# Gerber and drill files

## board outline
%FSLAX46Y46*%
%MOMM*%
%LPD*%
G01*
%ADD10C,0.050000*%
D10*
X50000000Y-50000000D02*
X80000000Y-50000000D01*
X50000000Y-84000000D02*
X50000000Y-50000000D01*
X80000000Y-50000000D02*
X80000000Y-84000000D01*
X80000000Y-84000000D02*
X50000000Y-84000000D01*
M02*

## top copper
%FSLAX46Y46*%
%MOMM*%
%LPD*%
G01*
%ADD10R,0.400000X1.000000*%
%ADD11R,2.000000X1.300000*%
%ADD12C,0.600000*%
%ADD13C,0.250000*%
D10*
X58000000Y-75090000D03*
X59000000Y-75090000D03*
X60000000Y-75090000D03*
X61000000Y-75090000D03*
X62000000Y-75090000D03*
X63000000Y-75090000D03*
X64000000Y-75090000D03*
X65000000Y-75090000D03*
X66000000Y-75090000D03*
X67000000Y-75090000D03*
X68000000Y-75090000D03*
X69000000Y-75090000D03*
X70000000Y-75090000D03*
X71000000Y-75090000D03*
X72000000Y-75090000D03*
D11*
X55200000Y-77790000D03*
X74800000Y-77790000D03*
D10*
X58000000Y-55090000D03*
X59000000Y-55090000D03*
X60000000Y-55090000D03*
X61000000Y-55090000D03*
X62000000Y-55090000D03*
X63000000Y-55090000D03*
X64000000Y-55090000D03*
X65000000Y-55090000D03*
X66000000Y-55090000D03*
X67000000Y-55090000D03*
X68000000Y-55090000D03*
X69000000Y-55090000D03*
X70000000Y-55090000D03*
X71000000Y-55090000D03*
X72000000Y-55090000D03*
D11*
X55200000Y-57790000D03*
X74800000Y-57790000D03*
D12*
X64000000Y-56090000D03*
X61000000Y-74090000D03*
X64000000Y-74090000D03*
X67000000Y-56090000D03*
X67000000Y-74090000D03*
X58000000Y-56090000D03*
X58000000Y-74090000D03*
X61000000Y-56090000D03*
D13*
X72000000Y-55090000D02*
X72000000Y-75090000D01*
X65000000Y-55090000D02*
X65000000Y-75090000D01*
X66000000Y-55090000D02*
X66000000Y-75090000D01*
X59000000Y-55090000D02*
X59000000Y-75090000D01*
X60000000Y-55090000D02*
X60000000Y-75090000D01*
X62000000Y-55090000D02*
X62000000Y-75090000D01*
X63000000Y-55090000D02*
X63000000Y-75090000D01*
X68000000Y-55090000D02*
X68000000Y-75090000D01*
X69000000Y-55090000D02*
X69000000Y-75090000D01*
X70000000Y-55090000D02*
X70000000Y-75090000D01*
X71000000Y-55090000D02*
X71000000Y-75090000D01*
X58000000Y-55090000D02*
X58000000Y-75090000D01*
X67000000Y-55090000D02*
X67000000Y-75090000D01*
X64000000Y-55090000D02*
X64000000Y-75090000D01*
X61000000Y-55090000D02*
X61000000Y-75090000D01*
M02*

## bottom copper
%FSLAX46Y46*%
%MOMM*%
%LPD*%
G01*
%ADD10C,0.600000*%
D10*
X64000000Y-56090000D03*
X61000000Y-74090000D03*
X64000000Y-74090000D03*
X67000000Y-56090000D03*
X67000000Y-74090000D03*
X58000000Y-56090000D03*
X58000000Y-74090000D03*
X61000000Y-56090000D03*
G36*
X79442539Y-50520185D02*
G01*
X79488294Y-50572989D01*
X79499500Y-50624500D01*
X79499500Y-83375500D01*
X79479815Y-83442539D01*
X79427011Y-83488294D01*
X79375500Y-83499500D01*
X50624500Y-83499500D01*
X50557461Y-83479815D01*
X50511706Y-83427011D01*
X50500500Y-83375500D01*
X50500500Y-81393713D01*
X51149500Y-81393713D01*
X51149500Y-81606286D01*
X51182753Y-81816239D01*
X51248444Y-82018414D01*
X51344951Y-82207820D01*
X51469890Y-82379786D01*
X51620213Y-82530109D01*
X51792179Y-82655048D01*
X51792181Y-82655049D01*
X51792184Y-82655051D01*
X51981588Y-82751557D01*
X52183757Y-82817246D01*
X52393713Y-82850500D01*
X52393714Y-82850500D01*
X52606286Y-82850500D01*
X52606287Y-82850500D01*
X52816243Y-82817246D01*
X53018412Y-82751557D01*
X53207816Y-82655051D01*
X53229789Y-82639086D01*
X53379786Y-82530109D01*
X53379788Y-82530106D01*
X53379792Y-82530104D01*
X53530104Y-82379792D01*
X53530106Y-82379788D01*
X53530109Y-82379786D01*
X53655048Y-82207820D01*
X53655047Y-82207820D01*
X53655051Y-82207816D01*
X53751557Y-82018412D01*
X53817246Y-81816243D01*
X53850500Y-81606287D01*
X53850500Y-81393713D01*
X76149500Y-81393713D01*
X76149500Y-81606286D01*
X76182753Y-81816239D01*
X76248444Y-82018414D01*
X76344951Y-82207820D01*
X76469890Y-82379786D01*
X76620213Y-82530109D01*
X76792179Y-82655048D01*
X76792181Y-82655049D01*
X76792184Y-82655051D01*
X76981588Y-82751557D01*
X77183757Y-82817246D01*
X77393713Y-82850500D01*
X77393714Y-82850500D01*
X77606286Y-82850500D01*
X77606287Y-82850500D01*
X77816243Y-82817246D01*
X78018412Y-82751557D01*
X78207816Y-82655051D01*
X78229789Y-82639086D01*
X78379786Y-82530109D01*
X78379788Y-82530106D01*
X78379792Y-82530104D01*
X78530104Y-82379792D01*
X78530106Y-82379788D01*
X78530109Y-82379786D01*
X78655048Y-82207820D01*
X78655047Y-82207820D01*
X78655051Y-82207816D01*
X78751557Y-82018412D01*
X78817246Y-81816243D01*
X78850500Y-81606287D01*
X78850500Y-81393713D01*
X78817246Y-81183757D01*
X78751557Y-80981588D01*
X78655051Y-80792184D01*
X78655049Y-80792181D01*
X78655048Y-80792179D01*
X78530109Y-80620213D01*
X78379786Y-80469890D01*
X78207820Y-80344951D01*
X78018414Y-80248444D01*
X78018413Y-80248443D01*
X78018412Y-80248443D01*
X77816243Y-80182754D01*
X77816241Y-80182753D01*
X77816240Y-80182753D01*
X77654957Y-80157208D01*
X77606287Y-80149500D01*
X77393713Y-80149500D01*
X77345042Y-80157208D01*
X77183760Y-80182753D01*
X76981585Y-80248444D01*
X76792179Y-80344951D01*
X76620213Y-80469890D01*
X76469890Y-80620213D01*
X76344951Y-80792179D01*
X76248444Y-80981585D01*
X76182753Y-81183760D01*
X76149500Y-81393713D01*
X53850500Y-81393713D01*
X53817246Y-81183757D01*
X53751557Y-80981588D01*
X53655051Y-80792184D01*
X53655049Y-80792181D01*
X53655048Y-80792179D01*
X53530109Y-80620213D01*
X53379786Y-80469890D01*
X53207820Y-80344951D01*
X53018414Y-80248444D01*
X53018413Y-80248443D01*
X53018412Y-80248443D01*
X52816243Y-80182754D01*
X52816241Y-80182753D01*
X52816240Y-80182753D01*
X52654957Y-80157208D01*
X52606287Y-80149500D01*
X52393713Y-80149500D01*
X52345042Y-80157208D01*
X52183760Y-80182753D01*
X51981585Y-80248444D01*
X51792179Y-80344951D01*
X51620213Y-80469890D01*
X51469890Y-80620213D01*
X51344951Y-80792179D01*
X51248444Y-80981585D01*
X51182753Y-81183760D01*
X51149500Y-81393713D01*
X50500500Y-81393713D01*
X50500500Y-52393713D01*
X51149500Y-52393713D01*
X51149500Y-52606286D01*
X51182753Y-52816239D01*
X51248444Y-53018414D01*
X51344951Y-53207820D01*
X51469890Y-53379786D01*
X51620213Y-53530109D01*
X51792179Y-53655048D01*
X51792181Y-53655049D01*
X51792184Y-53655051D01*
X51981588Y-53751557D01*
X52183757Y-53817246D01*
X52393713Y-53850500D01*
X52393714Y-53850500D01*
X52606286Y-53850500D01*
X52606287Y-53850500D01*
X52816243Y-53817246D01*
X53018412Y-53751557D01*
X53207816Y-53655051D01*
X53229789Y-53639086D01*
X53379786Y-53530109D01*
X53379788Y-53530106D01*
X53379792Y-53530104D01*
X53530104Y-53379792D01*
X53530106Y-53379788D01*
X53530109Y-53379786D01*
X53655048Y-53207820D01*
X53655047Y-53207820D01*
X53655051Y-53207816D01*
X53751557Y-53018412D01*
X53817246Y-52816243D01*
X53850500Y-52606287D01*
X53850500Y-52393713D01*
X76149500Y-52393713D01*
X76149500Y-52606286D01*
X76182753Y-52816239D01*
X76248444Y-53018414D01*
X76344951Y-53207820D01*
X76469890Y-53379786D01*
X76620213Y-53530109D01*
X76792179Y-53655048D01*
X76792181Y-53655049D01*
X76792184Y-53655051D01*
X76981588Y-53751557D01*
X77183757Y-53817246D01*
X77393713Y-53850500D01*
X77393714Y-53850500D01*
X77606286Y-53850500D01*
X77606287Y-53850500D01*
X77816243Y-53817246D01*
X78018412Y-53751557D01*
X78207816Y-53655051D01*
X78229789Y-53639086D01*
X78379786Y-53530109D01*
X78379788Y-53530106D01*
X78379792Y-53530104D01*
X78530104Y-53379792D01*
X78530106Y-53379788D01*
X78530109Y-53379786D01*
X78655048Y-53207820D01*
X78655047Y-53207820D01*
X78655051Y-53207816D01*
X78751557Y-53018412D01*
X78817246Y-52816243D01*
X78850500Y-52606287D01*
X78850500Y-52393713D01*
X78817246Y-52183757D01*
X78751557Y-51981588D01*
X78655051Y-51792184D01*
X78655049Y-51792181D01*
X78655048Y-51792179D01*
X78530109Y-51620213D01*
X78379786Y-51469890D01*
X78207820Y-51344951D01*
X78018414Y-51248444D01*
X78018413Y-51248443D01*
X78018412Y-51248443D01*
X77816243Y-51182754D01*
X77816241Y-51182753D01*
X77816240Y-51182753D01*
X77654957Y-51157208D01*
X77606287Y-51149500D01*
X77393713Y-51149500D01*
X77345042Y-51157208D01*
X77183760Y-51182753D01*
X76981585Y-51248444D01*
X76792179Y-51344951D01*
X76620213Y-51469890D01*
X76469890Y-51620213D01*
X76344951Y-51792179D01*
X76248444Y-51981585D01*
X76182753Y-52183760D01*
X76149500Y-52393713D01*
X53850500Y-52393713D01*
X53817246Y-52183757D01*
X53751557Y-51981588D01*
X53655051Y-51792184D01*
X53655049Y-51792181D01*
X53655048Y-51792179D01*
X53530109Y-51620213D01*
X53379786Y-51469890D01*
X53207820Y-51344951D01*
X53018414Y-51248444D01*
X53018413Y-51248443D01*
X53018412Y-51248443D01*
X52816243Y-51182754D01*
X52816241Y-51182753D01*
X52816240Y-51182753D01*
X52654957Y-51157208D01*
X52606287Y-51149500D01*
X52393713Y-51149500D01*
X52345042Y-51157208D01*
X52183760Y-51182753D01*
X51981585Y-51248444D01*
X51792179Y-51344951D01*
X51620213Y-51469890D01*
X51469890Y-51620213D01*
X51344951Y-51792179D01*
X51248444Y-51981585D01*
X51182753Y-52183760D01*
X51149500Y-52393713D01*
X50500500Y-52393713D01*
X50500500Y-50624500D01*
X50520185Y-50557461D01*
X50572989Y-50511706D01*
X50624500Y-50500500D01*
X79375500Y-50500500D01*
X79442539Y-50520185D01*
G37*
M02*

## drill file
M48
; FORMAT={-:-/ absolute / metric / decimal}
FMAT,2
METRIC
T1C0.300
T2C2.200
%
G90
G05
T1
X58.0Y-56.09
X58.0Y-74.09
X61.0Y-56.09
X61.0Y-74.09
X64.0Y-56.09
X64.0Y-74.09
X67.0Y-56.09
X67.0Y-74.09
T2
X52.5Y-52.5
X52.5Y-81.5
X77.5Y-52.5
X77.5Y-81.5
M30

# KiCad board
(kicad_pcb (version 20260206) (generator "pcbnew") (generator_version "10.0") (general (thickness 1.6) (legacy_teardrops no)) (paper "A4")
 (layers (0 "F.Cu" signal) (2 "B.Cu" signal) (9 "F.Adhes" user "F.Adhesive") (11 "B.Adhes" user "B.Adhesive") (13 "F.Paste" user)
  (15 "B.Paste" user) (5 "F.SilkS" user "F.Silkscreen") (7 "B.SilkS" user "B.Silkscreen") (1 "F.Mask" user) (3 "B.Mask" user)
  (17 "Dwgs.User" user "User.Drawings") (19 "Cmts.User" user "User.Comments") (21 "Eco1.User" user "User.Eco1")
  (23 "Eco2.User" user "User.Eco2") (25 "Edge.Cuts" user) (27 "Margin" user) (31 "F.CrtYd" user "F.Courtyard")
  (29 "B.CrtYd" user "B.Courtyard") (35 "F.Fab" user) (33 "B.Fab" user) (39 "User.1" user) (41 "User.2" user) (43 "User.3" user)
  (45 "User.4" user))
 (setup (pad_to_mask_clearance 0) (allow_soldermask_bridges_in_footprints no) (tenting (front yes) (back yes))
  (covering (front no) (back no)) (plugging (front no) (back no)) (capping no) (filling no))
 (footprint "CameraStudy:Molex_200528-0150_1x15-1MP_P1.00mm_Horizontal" (layer "F.Cu") (at 65 76)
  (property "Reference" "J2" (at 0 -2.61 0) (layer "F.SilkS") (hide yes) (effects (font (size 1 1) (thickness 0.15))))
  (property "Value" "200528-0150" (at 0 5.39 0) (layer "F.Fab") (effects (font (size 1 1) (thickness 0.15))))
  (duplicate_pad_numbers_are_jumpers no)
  (pad "1" smd rect (at -7 -0.91) (size 0.4 1) (layers "F.Cu" "F.Mask" "F.Paste") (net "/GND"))
  (pad "2" smd rect (at -6 -0.91) (size 0.4 1) (layers "F.Cu" "F.Mask" "F.Paste") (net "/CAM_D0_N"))
  (pad "3" smd rect (at -5 -0.91) (size 0.4 1) (layers "F.Cu" "F.Mask" "F.Paste") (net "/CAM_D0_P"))
  (pad "4" smd rect (at -4 -0.91) (size 0.4 1) (layers "F.Cu" "F.Mask" "F.Paste") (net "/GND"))
  (pad "5" smd rect (at -3 -0.91) (size 0.4 1) (layers "F.Cu" "F.Mask" "F.Paste") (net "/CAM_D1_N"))
  (pad "6" smd rect (at -2 -0.91) (size 0.4 1) (layers "F.Cu" "F.Mask" "F.Paste") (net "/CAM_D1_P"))
  (pad "7" smd rect (at -1 -0.91) (size 0.4 1) (layers "F.Cu" "F.Mask" "F.Paste") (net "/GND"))
  (pad "8" smd rect (at 0 -0.91) (size 0.4 1) (layers "F.Cu" "F.Mask" "F.Paste") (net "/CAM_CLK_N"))
  (pad "9" smd rect (at 1 -0.91) (size 0.4 1) (layers "F.Cu" "F.Mask" "F.Paste") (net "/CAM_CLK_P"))
  (pad "10" smd rect (at 2 -0.91) (size 0.4 1) (layers "F.Cu" "F.Mask" "F.Paste") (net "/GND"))
  (pad "11" smd rect (at 3 -0.91) (size 0.4 1) (layers "F.Cu" "F.Mask" "F.Paste") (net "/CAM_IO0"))
  (pad "12" smd rect (at 4 -0.91) (size 0.4 1) (layers "F.Cu" "F.Mask" "F.Paste") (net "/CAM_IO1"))
  (pad "13" smd rect (at 5 -0.91) (size 0.4 1) (layers "F.Cu" "F.Mask" "F.Paste") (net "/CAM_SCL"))
  (pad "14" smd rect (at 6 -0.91) (size 0.4 1) (layers "F.Cu" "F.Mask" "F.Paste") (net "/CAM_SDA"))
  (pad "15" smd rect (at 7 -0.91) (size 0.4 1) (layers "F.Cu" "F.Mask" "F.Paste") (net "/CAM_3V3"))
  (pad "MP" smd rect (at -9.8 1.79) (size 2 1.3) (layers "F.Cu" "F.Mask" "F.Paste"))
  (pad "MP" smd rect (at 9.8 1.79) (size 2 1.3) (layers "F.Cu" "F.Mask" "F.Paste")))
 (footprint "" (layer "F.Cu") (at 77.5 52.5)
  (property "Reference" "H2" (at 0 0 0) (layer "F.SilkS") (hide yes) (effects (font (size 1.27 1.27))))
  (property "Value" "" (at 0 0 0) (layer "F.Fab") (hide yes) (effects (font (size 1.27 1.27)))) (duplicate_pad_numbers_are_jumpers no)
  (pad "" np_thru_hole circle (at 0 0) (size 2.2 2.2) (drill 2.2) (layers "*.Cu")))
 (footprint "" (layer "F.Cu") (at 77.5 81.5)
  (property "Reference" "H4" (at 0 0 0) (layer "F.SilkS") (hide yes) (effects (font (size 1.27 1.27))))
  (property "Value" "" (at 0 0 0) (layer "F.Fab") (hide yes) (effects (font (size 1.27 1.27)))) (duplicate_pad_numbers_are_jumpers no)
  (pad "" np_thru_hole circle (at 0 0) (size 2.2 2.2) (drill 2.2) (layers "*.Cu")))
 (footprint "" (layer "F.Cu") (at 52.5 52.5)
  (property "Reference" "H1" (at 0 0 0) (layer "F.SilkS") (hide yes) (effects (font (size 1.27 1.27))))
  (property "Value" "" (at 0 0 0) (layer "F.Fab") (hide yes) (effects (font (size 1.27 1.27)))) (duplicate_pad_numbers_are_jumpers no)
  (pad "" np_thru_hole circle (at 0 0) (size 2.2 2.2) (drill 2.2) (layers "*.Cu")))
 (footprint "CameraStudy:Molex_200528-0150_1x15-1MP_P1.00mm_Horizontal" (layer "F.Cu") (at 65 56)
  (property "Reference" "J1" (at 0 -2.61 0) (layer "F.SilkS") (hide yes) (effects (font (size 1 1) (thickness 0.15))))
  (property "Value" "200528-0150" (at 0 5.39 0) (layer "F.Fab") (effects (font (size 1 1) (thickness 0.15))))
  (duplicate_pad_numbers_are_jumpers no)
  (pad "1" smd rect (at -7 -0.91) (size 0.4 1) (layers "F.Cu" "F.Mask" "F.Paste") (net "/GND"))
  (pad "2" smd rect (at -6 -0.91) (size 0.4 1) (layers "F.Cu" "F.Mask" "F.Paste") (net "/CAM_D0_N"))
  (pad "3" smd rect (at -5 -0.91) (size 0.4 1) (layers "F.Cu" "F.Mask" "F.Paste") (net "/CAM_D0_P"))
  (pad "4" smd rect (at -4 -0.91) (size 0.4 1) (layers "F.Cu" "F.Mask" "F.Paste") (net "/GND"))
  (pad "5" smd rect (at -3 -0.91) (size 0.4 1) (layers "F.Cu" "F.Mask" "F.Paste") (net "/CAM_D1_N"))
  (pad "6" smd rect (at -2 -0.91) (size 0.4 1) (layers "F.Cu" "F.Mask" "F.Paste") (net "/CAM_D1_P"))
  (pad "7" smd rect (at -1 -0.91) (size 0.4 1) (layers "F.Cu" "F.Mask" "F.Paste") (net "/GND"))
  (pad "8" smd rect (at 0 -0.91) (size 0.4 1) (layers "F.Cu" "F.Mask" "F.Paste") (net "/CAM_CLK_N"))
  (pad "9" smd rect (at 1 -0.91) (size 0.4 1) (layers "F.Cu" "F.Mask" "F.Paste") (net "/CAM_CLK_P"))
  (pad "10" smd rect (at 2 -0.91) (size 0.4 1) (layers "F.Cu" "F.Mask" "F.Paste") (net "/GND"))
  (pad "11" smd rect (at 3 -0.91) (size 0.4 1) (layers "F.Cu" "F.Mask" "F.Paste") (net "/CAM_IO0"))
  (pad "12" smd rect (at 4 -0.91) (size 0.4 1) (layers "F.Cu" "F.Mask" "F.Paste") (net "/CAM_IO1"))
  (pad "13" smd rect (at 5 -0.91) (size 0.4 1) (layers "F.Cu" "F.Mask" "F.Paste") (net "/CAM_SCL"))
  (pad "14" smd rect (at 6 -0.91) (size 0.4 1) (layers "F.Cu" "F.Mask" "F.Paste") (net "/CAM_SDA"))
  (pad "15" smd rect (at 7 -0.91) (size 0.4 1) (layers "F.Cu" "F.Mask" "F.Paste") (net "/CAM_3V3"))
  (pad "MP" smd rect (at -9.8 1.79) (size 2 1.3) (layers "F.Cu" "F.Mask" "F.Paste"))
  (pad "MP" smd rect (at 9.8 1.79) (size 2 1.3) (layers "F.Cu" "F.Mask" "F.Paste")))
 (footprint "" (layer "F.Cu") (at 52.5 81.5)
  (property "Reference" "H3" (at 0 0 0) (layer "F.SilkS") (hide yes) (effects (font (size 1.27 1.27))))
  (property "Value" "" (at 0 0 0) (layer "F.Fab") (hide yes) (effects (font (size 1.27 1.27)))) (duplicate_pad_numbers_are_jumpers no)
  (pad "" np_thru_hole circle (at 0 0) (size 2.2 2.2) (drill 2.2) (layers "*.Cu")))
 (gr_line (start 50 50) (end 80 50) (stroke (width 0.05) (type default)) (layer "Edge.Cuts"))
 (gr_line (start 50 84) (end 50 50) (stroke (width 0.05) (type default)) (layer "Edge.Cuts"))
 (gr_line (start 80 50) (end 80 84) (stroke (width 0.05) (type default)) (layer "Edge.Cuts"))
 (gr_line (start 80 84) (end 50 84) (stroke (width 0.05) (type default)) (layer "Edge.Cuts"))
 (segment (start 72 55.09) (end 72 75.09) (width 0.25) (layer "F.Cu") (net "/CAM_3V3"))
 (segment (start 65 55.09) (end 65 75.09) (width 0.25) (layer "F.Cu") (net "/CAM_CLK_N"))
 (segment (start 66 55.09) (end 66 75.09) (width 0.25) (layer "F.Cu") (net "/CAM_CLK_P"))
 (segment (start 59 55.09) (end 59 75.09) (width 0.25) (layer "F.Cu") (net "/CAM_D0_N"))
 (segment (start 60 55.09) (end 60 75.09) (width 0.25) (layer "F.Cu") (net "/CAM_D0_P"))
 (segment (start 62 55.09) (end 62 75.09) (width 0.25) (layer "F.Cu") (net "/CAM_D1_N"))
 (segment (start 63 55.09) (end 63 75.09) (width 0.25) (layer "F.Cu") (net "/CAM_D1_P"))
 (segment (start 68 55.09) (end 68 75.09) (width 0.25) (layer "F.Cu") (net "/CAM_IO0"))
 (segment (start 69 55.09) (end 69 75.09) (width 0.25) (layer "F.Cu") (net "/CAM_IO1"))
 (segment (start 70 55.09) (end 70 75.09) (width 0.25) (layer "F.Cu") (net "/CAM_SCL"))
 (segment (start 71 55.09) (end 71 75.09) (width 0.25) (layer "F.Cu") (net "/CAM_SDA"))
 (segment (start 58 55.09) (end 58 75.09) (width 0.25) (layer "F.Cu") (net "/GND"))
 (segment (start 67 55.09) (end 67 75.09) (width 0.25) (layer "F.Cu") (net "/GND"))
 (segment (start 64 55.09) (end 64 75.09) (width 0.25) (layer "F.Cu") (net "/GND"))
 (segment (start 61 55.09) (end 61 75.09) (width 0.25) (layer "F.Cu") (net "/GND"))
 (via (at 64 56.09) (size 0.6) (drill 0.3) (layers "F.Cu" "B.Cu") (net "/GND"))
 (via (at 61 74.09) (size 0.6) (drill 0.3) (layers "F.Cu" "B.Cu") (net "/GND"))
 (via (at 64 74.09) (size 0.6) (drill 0.3) (layers "F.Cu" "B.Cu") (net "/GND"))
 (via (at 67 56.09) (size 0.6) (drill 0.3) (layers "F.Cu" "B.Cu") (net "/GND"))
 (via (at 67 74.09) (size 0.6) (drill 0.3) (layers "F.Cu" "B.Cu") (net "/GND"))
 (via (at 58 56.09) (size 0.6) (drill 0.3) (layers "F.Cu" "B.Cu") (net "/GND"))
 (via (at 58 74.09) (size 0.6) (drill 0.3) (layers "F.Cu" "B.Cu") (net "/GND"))
 (via (at 61 56.09) (size 0.6) (drill 0.3) (layers "F.Cu" "B.Cu") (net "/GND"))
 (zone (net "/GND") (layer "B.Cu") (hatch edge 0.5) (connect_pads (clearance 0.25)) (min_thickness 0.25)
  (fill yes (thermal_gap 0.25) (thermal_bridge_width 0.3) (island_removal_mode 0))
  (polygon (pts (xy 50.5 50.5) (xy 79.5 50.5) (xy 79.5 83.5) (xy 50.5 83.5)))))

